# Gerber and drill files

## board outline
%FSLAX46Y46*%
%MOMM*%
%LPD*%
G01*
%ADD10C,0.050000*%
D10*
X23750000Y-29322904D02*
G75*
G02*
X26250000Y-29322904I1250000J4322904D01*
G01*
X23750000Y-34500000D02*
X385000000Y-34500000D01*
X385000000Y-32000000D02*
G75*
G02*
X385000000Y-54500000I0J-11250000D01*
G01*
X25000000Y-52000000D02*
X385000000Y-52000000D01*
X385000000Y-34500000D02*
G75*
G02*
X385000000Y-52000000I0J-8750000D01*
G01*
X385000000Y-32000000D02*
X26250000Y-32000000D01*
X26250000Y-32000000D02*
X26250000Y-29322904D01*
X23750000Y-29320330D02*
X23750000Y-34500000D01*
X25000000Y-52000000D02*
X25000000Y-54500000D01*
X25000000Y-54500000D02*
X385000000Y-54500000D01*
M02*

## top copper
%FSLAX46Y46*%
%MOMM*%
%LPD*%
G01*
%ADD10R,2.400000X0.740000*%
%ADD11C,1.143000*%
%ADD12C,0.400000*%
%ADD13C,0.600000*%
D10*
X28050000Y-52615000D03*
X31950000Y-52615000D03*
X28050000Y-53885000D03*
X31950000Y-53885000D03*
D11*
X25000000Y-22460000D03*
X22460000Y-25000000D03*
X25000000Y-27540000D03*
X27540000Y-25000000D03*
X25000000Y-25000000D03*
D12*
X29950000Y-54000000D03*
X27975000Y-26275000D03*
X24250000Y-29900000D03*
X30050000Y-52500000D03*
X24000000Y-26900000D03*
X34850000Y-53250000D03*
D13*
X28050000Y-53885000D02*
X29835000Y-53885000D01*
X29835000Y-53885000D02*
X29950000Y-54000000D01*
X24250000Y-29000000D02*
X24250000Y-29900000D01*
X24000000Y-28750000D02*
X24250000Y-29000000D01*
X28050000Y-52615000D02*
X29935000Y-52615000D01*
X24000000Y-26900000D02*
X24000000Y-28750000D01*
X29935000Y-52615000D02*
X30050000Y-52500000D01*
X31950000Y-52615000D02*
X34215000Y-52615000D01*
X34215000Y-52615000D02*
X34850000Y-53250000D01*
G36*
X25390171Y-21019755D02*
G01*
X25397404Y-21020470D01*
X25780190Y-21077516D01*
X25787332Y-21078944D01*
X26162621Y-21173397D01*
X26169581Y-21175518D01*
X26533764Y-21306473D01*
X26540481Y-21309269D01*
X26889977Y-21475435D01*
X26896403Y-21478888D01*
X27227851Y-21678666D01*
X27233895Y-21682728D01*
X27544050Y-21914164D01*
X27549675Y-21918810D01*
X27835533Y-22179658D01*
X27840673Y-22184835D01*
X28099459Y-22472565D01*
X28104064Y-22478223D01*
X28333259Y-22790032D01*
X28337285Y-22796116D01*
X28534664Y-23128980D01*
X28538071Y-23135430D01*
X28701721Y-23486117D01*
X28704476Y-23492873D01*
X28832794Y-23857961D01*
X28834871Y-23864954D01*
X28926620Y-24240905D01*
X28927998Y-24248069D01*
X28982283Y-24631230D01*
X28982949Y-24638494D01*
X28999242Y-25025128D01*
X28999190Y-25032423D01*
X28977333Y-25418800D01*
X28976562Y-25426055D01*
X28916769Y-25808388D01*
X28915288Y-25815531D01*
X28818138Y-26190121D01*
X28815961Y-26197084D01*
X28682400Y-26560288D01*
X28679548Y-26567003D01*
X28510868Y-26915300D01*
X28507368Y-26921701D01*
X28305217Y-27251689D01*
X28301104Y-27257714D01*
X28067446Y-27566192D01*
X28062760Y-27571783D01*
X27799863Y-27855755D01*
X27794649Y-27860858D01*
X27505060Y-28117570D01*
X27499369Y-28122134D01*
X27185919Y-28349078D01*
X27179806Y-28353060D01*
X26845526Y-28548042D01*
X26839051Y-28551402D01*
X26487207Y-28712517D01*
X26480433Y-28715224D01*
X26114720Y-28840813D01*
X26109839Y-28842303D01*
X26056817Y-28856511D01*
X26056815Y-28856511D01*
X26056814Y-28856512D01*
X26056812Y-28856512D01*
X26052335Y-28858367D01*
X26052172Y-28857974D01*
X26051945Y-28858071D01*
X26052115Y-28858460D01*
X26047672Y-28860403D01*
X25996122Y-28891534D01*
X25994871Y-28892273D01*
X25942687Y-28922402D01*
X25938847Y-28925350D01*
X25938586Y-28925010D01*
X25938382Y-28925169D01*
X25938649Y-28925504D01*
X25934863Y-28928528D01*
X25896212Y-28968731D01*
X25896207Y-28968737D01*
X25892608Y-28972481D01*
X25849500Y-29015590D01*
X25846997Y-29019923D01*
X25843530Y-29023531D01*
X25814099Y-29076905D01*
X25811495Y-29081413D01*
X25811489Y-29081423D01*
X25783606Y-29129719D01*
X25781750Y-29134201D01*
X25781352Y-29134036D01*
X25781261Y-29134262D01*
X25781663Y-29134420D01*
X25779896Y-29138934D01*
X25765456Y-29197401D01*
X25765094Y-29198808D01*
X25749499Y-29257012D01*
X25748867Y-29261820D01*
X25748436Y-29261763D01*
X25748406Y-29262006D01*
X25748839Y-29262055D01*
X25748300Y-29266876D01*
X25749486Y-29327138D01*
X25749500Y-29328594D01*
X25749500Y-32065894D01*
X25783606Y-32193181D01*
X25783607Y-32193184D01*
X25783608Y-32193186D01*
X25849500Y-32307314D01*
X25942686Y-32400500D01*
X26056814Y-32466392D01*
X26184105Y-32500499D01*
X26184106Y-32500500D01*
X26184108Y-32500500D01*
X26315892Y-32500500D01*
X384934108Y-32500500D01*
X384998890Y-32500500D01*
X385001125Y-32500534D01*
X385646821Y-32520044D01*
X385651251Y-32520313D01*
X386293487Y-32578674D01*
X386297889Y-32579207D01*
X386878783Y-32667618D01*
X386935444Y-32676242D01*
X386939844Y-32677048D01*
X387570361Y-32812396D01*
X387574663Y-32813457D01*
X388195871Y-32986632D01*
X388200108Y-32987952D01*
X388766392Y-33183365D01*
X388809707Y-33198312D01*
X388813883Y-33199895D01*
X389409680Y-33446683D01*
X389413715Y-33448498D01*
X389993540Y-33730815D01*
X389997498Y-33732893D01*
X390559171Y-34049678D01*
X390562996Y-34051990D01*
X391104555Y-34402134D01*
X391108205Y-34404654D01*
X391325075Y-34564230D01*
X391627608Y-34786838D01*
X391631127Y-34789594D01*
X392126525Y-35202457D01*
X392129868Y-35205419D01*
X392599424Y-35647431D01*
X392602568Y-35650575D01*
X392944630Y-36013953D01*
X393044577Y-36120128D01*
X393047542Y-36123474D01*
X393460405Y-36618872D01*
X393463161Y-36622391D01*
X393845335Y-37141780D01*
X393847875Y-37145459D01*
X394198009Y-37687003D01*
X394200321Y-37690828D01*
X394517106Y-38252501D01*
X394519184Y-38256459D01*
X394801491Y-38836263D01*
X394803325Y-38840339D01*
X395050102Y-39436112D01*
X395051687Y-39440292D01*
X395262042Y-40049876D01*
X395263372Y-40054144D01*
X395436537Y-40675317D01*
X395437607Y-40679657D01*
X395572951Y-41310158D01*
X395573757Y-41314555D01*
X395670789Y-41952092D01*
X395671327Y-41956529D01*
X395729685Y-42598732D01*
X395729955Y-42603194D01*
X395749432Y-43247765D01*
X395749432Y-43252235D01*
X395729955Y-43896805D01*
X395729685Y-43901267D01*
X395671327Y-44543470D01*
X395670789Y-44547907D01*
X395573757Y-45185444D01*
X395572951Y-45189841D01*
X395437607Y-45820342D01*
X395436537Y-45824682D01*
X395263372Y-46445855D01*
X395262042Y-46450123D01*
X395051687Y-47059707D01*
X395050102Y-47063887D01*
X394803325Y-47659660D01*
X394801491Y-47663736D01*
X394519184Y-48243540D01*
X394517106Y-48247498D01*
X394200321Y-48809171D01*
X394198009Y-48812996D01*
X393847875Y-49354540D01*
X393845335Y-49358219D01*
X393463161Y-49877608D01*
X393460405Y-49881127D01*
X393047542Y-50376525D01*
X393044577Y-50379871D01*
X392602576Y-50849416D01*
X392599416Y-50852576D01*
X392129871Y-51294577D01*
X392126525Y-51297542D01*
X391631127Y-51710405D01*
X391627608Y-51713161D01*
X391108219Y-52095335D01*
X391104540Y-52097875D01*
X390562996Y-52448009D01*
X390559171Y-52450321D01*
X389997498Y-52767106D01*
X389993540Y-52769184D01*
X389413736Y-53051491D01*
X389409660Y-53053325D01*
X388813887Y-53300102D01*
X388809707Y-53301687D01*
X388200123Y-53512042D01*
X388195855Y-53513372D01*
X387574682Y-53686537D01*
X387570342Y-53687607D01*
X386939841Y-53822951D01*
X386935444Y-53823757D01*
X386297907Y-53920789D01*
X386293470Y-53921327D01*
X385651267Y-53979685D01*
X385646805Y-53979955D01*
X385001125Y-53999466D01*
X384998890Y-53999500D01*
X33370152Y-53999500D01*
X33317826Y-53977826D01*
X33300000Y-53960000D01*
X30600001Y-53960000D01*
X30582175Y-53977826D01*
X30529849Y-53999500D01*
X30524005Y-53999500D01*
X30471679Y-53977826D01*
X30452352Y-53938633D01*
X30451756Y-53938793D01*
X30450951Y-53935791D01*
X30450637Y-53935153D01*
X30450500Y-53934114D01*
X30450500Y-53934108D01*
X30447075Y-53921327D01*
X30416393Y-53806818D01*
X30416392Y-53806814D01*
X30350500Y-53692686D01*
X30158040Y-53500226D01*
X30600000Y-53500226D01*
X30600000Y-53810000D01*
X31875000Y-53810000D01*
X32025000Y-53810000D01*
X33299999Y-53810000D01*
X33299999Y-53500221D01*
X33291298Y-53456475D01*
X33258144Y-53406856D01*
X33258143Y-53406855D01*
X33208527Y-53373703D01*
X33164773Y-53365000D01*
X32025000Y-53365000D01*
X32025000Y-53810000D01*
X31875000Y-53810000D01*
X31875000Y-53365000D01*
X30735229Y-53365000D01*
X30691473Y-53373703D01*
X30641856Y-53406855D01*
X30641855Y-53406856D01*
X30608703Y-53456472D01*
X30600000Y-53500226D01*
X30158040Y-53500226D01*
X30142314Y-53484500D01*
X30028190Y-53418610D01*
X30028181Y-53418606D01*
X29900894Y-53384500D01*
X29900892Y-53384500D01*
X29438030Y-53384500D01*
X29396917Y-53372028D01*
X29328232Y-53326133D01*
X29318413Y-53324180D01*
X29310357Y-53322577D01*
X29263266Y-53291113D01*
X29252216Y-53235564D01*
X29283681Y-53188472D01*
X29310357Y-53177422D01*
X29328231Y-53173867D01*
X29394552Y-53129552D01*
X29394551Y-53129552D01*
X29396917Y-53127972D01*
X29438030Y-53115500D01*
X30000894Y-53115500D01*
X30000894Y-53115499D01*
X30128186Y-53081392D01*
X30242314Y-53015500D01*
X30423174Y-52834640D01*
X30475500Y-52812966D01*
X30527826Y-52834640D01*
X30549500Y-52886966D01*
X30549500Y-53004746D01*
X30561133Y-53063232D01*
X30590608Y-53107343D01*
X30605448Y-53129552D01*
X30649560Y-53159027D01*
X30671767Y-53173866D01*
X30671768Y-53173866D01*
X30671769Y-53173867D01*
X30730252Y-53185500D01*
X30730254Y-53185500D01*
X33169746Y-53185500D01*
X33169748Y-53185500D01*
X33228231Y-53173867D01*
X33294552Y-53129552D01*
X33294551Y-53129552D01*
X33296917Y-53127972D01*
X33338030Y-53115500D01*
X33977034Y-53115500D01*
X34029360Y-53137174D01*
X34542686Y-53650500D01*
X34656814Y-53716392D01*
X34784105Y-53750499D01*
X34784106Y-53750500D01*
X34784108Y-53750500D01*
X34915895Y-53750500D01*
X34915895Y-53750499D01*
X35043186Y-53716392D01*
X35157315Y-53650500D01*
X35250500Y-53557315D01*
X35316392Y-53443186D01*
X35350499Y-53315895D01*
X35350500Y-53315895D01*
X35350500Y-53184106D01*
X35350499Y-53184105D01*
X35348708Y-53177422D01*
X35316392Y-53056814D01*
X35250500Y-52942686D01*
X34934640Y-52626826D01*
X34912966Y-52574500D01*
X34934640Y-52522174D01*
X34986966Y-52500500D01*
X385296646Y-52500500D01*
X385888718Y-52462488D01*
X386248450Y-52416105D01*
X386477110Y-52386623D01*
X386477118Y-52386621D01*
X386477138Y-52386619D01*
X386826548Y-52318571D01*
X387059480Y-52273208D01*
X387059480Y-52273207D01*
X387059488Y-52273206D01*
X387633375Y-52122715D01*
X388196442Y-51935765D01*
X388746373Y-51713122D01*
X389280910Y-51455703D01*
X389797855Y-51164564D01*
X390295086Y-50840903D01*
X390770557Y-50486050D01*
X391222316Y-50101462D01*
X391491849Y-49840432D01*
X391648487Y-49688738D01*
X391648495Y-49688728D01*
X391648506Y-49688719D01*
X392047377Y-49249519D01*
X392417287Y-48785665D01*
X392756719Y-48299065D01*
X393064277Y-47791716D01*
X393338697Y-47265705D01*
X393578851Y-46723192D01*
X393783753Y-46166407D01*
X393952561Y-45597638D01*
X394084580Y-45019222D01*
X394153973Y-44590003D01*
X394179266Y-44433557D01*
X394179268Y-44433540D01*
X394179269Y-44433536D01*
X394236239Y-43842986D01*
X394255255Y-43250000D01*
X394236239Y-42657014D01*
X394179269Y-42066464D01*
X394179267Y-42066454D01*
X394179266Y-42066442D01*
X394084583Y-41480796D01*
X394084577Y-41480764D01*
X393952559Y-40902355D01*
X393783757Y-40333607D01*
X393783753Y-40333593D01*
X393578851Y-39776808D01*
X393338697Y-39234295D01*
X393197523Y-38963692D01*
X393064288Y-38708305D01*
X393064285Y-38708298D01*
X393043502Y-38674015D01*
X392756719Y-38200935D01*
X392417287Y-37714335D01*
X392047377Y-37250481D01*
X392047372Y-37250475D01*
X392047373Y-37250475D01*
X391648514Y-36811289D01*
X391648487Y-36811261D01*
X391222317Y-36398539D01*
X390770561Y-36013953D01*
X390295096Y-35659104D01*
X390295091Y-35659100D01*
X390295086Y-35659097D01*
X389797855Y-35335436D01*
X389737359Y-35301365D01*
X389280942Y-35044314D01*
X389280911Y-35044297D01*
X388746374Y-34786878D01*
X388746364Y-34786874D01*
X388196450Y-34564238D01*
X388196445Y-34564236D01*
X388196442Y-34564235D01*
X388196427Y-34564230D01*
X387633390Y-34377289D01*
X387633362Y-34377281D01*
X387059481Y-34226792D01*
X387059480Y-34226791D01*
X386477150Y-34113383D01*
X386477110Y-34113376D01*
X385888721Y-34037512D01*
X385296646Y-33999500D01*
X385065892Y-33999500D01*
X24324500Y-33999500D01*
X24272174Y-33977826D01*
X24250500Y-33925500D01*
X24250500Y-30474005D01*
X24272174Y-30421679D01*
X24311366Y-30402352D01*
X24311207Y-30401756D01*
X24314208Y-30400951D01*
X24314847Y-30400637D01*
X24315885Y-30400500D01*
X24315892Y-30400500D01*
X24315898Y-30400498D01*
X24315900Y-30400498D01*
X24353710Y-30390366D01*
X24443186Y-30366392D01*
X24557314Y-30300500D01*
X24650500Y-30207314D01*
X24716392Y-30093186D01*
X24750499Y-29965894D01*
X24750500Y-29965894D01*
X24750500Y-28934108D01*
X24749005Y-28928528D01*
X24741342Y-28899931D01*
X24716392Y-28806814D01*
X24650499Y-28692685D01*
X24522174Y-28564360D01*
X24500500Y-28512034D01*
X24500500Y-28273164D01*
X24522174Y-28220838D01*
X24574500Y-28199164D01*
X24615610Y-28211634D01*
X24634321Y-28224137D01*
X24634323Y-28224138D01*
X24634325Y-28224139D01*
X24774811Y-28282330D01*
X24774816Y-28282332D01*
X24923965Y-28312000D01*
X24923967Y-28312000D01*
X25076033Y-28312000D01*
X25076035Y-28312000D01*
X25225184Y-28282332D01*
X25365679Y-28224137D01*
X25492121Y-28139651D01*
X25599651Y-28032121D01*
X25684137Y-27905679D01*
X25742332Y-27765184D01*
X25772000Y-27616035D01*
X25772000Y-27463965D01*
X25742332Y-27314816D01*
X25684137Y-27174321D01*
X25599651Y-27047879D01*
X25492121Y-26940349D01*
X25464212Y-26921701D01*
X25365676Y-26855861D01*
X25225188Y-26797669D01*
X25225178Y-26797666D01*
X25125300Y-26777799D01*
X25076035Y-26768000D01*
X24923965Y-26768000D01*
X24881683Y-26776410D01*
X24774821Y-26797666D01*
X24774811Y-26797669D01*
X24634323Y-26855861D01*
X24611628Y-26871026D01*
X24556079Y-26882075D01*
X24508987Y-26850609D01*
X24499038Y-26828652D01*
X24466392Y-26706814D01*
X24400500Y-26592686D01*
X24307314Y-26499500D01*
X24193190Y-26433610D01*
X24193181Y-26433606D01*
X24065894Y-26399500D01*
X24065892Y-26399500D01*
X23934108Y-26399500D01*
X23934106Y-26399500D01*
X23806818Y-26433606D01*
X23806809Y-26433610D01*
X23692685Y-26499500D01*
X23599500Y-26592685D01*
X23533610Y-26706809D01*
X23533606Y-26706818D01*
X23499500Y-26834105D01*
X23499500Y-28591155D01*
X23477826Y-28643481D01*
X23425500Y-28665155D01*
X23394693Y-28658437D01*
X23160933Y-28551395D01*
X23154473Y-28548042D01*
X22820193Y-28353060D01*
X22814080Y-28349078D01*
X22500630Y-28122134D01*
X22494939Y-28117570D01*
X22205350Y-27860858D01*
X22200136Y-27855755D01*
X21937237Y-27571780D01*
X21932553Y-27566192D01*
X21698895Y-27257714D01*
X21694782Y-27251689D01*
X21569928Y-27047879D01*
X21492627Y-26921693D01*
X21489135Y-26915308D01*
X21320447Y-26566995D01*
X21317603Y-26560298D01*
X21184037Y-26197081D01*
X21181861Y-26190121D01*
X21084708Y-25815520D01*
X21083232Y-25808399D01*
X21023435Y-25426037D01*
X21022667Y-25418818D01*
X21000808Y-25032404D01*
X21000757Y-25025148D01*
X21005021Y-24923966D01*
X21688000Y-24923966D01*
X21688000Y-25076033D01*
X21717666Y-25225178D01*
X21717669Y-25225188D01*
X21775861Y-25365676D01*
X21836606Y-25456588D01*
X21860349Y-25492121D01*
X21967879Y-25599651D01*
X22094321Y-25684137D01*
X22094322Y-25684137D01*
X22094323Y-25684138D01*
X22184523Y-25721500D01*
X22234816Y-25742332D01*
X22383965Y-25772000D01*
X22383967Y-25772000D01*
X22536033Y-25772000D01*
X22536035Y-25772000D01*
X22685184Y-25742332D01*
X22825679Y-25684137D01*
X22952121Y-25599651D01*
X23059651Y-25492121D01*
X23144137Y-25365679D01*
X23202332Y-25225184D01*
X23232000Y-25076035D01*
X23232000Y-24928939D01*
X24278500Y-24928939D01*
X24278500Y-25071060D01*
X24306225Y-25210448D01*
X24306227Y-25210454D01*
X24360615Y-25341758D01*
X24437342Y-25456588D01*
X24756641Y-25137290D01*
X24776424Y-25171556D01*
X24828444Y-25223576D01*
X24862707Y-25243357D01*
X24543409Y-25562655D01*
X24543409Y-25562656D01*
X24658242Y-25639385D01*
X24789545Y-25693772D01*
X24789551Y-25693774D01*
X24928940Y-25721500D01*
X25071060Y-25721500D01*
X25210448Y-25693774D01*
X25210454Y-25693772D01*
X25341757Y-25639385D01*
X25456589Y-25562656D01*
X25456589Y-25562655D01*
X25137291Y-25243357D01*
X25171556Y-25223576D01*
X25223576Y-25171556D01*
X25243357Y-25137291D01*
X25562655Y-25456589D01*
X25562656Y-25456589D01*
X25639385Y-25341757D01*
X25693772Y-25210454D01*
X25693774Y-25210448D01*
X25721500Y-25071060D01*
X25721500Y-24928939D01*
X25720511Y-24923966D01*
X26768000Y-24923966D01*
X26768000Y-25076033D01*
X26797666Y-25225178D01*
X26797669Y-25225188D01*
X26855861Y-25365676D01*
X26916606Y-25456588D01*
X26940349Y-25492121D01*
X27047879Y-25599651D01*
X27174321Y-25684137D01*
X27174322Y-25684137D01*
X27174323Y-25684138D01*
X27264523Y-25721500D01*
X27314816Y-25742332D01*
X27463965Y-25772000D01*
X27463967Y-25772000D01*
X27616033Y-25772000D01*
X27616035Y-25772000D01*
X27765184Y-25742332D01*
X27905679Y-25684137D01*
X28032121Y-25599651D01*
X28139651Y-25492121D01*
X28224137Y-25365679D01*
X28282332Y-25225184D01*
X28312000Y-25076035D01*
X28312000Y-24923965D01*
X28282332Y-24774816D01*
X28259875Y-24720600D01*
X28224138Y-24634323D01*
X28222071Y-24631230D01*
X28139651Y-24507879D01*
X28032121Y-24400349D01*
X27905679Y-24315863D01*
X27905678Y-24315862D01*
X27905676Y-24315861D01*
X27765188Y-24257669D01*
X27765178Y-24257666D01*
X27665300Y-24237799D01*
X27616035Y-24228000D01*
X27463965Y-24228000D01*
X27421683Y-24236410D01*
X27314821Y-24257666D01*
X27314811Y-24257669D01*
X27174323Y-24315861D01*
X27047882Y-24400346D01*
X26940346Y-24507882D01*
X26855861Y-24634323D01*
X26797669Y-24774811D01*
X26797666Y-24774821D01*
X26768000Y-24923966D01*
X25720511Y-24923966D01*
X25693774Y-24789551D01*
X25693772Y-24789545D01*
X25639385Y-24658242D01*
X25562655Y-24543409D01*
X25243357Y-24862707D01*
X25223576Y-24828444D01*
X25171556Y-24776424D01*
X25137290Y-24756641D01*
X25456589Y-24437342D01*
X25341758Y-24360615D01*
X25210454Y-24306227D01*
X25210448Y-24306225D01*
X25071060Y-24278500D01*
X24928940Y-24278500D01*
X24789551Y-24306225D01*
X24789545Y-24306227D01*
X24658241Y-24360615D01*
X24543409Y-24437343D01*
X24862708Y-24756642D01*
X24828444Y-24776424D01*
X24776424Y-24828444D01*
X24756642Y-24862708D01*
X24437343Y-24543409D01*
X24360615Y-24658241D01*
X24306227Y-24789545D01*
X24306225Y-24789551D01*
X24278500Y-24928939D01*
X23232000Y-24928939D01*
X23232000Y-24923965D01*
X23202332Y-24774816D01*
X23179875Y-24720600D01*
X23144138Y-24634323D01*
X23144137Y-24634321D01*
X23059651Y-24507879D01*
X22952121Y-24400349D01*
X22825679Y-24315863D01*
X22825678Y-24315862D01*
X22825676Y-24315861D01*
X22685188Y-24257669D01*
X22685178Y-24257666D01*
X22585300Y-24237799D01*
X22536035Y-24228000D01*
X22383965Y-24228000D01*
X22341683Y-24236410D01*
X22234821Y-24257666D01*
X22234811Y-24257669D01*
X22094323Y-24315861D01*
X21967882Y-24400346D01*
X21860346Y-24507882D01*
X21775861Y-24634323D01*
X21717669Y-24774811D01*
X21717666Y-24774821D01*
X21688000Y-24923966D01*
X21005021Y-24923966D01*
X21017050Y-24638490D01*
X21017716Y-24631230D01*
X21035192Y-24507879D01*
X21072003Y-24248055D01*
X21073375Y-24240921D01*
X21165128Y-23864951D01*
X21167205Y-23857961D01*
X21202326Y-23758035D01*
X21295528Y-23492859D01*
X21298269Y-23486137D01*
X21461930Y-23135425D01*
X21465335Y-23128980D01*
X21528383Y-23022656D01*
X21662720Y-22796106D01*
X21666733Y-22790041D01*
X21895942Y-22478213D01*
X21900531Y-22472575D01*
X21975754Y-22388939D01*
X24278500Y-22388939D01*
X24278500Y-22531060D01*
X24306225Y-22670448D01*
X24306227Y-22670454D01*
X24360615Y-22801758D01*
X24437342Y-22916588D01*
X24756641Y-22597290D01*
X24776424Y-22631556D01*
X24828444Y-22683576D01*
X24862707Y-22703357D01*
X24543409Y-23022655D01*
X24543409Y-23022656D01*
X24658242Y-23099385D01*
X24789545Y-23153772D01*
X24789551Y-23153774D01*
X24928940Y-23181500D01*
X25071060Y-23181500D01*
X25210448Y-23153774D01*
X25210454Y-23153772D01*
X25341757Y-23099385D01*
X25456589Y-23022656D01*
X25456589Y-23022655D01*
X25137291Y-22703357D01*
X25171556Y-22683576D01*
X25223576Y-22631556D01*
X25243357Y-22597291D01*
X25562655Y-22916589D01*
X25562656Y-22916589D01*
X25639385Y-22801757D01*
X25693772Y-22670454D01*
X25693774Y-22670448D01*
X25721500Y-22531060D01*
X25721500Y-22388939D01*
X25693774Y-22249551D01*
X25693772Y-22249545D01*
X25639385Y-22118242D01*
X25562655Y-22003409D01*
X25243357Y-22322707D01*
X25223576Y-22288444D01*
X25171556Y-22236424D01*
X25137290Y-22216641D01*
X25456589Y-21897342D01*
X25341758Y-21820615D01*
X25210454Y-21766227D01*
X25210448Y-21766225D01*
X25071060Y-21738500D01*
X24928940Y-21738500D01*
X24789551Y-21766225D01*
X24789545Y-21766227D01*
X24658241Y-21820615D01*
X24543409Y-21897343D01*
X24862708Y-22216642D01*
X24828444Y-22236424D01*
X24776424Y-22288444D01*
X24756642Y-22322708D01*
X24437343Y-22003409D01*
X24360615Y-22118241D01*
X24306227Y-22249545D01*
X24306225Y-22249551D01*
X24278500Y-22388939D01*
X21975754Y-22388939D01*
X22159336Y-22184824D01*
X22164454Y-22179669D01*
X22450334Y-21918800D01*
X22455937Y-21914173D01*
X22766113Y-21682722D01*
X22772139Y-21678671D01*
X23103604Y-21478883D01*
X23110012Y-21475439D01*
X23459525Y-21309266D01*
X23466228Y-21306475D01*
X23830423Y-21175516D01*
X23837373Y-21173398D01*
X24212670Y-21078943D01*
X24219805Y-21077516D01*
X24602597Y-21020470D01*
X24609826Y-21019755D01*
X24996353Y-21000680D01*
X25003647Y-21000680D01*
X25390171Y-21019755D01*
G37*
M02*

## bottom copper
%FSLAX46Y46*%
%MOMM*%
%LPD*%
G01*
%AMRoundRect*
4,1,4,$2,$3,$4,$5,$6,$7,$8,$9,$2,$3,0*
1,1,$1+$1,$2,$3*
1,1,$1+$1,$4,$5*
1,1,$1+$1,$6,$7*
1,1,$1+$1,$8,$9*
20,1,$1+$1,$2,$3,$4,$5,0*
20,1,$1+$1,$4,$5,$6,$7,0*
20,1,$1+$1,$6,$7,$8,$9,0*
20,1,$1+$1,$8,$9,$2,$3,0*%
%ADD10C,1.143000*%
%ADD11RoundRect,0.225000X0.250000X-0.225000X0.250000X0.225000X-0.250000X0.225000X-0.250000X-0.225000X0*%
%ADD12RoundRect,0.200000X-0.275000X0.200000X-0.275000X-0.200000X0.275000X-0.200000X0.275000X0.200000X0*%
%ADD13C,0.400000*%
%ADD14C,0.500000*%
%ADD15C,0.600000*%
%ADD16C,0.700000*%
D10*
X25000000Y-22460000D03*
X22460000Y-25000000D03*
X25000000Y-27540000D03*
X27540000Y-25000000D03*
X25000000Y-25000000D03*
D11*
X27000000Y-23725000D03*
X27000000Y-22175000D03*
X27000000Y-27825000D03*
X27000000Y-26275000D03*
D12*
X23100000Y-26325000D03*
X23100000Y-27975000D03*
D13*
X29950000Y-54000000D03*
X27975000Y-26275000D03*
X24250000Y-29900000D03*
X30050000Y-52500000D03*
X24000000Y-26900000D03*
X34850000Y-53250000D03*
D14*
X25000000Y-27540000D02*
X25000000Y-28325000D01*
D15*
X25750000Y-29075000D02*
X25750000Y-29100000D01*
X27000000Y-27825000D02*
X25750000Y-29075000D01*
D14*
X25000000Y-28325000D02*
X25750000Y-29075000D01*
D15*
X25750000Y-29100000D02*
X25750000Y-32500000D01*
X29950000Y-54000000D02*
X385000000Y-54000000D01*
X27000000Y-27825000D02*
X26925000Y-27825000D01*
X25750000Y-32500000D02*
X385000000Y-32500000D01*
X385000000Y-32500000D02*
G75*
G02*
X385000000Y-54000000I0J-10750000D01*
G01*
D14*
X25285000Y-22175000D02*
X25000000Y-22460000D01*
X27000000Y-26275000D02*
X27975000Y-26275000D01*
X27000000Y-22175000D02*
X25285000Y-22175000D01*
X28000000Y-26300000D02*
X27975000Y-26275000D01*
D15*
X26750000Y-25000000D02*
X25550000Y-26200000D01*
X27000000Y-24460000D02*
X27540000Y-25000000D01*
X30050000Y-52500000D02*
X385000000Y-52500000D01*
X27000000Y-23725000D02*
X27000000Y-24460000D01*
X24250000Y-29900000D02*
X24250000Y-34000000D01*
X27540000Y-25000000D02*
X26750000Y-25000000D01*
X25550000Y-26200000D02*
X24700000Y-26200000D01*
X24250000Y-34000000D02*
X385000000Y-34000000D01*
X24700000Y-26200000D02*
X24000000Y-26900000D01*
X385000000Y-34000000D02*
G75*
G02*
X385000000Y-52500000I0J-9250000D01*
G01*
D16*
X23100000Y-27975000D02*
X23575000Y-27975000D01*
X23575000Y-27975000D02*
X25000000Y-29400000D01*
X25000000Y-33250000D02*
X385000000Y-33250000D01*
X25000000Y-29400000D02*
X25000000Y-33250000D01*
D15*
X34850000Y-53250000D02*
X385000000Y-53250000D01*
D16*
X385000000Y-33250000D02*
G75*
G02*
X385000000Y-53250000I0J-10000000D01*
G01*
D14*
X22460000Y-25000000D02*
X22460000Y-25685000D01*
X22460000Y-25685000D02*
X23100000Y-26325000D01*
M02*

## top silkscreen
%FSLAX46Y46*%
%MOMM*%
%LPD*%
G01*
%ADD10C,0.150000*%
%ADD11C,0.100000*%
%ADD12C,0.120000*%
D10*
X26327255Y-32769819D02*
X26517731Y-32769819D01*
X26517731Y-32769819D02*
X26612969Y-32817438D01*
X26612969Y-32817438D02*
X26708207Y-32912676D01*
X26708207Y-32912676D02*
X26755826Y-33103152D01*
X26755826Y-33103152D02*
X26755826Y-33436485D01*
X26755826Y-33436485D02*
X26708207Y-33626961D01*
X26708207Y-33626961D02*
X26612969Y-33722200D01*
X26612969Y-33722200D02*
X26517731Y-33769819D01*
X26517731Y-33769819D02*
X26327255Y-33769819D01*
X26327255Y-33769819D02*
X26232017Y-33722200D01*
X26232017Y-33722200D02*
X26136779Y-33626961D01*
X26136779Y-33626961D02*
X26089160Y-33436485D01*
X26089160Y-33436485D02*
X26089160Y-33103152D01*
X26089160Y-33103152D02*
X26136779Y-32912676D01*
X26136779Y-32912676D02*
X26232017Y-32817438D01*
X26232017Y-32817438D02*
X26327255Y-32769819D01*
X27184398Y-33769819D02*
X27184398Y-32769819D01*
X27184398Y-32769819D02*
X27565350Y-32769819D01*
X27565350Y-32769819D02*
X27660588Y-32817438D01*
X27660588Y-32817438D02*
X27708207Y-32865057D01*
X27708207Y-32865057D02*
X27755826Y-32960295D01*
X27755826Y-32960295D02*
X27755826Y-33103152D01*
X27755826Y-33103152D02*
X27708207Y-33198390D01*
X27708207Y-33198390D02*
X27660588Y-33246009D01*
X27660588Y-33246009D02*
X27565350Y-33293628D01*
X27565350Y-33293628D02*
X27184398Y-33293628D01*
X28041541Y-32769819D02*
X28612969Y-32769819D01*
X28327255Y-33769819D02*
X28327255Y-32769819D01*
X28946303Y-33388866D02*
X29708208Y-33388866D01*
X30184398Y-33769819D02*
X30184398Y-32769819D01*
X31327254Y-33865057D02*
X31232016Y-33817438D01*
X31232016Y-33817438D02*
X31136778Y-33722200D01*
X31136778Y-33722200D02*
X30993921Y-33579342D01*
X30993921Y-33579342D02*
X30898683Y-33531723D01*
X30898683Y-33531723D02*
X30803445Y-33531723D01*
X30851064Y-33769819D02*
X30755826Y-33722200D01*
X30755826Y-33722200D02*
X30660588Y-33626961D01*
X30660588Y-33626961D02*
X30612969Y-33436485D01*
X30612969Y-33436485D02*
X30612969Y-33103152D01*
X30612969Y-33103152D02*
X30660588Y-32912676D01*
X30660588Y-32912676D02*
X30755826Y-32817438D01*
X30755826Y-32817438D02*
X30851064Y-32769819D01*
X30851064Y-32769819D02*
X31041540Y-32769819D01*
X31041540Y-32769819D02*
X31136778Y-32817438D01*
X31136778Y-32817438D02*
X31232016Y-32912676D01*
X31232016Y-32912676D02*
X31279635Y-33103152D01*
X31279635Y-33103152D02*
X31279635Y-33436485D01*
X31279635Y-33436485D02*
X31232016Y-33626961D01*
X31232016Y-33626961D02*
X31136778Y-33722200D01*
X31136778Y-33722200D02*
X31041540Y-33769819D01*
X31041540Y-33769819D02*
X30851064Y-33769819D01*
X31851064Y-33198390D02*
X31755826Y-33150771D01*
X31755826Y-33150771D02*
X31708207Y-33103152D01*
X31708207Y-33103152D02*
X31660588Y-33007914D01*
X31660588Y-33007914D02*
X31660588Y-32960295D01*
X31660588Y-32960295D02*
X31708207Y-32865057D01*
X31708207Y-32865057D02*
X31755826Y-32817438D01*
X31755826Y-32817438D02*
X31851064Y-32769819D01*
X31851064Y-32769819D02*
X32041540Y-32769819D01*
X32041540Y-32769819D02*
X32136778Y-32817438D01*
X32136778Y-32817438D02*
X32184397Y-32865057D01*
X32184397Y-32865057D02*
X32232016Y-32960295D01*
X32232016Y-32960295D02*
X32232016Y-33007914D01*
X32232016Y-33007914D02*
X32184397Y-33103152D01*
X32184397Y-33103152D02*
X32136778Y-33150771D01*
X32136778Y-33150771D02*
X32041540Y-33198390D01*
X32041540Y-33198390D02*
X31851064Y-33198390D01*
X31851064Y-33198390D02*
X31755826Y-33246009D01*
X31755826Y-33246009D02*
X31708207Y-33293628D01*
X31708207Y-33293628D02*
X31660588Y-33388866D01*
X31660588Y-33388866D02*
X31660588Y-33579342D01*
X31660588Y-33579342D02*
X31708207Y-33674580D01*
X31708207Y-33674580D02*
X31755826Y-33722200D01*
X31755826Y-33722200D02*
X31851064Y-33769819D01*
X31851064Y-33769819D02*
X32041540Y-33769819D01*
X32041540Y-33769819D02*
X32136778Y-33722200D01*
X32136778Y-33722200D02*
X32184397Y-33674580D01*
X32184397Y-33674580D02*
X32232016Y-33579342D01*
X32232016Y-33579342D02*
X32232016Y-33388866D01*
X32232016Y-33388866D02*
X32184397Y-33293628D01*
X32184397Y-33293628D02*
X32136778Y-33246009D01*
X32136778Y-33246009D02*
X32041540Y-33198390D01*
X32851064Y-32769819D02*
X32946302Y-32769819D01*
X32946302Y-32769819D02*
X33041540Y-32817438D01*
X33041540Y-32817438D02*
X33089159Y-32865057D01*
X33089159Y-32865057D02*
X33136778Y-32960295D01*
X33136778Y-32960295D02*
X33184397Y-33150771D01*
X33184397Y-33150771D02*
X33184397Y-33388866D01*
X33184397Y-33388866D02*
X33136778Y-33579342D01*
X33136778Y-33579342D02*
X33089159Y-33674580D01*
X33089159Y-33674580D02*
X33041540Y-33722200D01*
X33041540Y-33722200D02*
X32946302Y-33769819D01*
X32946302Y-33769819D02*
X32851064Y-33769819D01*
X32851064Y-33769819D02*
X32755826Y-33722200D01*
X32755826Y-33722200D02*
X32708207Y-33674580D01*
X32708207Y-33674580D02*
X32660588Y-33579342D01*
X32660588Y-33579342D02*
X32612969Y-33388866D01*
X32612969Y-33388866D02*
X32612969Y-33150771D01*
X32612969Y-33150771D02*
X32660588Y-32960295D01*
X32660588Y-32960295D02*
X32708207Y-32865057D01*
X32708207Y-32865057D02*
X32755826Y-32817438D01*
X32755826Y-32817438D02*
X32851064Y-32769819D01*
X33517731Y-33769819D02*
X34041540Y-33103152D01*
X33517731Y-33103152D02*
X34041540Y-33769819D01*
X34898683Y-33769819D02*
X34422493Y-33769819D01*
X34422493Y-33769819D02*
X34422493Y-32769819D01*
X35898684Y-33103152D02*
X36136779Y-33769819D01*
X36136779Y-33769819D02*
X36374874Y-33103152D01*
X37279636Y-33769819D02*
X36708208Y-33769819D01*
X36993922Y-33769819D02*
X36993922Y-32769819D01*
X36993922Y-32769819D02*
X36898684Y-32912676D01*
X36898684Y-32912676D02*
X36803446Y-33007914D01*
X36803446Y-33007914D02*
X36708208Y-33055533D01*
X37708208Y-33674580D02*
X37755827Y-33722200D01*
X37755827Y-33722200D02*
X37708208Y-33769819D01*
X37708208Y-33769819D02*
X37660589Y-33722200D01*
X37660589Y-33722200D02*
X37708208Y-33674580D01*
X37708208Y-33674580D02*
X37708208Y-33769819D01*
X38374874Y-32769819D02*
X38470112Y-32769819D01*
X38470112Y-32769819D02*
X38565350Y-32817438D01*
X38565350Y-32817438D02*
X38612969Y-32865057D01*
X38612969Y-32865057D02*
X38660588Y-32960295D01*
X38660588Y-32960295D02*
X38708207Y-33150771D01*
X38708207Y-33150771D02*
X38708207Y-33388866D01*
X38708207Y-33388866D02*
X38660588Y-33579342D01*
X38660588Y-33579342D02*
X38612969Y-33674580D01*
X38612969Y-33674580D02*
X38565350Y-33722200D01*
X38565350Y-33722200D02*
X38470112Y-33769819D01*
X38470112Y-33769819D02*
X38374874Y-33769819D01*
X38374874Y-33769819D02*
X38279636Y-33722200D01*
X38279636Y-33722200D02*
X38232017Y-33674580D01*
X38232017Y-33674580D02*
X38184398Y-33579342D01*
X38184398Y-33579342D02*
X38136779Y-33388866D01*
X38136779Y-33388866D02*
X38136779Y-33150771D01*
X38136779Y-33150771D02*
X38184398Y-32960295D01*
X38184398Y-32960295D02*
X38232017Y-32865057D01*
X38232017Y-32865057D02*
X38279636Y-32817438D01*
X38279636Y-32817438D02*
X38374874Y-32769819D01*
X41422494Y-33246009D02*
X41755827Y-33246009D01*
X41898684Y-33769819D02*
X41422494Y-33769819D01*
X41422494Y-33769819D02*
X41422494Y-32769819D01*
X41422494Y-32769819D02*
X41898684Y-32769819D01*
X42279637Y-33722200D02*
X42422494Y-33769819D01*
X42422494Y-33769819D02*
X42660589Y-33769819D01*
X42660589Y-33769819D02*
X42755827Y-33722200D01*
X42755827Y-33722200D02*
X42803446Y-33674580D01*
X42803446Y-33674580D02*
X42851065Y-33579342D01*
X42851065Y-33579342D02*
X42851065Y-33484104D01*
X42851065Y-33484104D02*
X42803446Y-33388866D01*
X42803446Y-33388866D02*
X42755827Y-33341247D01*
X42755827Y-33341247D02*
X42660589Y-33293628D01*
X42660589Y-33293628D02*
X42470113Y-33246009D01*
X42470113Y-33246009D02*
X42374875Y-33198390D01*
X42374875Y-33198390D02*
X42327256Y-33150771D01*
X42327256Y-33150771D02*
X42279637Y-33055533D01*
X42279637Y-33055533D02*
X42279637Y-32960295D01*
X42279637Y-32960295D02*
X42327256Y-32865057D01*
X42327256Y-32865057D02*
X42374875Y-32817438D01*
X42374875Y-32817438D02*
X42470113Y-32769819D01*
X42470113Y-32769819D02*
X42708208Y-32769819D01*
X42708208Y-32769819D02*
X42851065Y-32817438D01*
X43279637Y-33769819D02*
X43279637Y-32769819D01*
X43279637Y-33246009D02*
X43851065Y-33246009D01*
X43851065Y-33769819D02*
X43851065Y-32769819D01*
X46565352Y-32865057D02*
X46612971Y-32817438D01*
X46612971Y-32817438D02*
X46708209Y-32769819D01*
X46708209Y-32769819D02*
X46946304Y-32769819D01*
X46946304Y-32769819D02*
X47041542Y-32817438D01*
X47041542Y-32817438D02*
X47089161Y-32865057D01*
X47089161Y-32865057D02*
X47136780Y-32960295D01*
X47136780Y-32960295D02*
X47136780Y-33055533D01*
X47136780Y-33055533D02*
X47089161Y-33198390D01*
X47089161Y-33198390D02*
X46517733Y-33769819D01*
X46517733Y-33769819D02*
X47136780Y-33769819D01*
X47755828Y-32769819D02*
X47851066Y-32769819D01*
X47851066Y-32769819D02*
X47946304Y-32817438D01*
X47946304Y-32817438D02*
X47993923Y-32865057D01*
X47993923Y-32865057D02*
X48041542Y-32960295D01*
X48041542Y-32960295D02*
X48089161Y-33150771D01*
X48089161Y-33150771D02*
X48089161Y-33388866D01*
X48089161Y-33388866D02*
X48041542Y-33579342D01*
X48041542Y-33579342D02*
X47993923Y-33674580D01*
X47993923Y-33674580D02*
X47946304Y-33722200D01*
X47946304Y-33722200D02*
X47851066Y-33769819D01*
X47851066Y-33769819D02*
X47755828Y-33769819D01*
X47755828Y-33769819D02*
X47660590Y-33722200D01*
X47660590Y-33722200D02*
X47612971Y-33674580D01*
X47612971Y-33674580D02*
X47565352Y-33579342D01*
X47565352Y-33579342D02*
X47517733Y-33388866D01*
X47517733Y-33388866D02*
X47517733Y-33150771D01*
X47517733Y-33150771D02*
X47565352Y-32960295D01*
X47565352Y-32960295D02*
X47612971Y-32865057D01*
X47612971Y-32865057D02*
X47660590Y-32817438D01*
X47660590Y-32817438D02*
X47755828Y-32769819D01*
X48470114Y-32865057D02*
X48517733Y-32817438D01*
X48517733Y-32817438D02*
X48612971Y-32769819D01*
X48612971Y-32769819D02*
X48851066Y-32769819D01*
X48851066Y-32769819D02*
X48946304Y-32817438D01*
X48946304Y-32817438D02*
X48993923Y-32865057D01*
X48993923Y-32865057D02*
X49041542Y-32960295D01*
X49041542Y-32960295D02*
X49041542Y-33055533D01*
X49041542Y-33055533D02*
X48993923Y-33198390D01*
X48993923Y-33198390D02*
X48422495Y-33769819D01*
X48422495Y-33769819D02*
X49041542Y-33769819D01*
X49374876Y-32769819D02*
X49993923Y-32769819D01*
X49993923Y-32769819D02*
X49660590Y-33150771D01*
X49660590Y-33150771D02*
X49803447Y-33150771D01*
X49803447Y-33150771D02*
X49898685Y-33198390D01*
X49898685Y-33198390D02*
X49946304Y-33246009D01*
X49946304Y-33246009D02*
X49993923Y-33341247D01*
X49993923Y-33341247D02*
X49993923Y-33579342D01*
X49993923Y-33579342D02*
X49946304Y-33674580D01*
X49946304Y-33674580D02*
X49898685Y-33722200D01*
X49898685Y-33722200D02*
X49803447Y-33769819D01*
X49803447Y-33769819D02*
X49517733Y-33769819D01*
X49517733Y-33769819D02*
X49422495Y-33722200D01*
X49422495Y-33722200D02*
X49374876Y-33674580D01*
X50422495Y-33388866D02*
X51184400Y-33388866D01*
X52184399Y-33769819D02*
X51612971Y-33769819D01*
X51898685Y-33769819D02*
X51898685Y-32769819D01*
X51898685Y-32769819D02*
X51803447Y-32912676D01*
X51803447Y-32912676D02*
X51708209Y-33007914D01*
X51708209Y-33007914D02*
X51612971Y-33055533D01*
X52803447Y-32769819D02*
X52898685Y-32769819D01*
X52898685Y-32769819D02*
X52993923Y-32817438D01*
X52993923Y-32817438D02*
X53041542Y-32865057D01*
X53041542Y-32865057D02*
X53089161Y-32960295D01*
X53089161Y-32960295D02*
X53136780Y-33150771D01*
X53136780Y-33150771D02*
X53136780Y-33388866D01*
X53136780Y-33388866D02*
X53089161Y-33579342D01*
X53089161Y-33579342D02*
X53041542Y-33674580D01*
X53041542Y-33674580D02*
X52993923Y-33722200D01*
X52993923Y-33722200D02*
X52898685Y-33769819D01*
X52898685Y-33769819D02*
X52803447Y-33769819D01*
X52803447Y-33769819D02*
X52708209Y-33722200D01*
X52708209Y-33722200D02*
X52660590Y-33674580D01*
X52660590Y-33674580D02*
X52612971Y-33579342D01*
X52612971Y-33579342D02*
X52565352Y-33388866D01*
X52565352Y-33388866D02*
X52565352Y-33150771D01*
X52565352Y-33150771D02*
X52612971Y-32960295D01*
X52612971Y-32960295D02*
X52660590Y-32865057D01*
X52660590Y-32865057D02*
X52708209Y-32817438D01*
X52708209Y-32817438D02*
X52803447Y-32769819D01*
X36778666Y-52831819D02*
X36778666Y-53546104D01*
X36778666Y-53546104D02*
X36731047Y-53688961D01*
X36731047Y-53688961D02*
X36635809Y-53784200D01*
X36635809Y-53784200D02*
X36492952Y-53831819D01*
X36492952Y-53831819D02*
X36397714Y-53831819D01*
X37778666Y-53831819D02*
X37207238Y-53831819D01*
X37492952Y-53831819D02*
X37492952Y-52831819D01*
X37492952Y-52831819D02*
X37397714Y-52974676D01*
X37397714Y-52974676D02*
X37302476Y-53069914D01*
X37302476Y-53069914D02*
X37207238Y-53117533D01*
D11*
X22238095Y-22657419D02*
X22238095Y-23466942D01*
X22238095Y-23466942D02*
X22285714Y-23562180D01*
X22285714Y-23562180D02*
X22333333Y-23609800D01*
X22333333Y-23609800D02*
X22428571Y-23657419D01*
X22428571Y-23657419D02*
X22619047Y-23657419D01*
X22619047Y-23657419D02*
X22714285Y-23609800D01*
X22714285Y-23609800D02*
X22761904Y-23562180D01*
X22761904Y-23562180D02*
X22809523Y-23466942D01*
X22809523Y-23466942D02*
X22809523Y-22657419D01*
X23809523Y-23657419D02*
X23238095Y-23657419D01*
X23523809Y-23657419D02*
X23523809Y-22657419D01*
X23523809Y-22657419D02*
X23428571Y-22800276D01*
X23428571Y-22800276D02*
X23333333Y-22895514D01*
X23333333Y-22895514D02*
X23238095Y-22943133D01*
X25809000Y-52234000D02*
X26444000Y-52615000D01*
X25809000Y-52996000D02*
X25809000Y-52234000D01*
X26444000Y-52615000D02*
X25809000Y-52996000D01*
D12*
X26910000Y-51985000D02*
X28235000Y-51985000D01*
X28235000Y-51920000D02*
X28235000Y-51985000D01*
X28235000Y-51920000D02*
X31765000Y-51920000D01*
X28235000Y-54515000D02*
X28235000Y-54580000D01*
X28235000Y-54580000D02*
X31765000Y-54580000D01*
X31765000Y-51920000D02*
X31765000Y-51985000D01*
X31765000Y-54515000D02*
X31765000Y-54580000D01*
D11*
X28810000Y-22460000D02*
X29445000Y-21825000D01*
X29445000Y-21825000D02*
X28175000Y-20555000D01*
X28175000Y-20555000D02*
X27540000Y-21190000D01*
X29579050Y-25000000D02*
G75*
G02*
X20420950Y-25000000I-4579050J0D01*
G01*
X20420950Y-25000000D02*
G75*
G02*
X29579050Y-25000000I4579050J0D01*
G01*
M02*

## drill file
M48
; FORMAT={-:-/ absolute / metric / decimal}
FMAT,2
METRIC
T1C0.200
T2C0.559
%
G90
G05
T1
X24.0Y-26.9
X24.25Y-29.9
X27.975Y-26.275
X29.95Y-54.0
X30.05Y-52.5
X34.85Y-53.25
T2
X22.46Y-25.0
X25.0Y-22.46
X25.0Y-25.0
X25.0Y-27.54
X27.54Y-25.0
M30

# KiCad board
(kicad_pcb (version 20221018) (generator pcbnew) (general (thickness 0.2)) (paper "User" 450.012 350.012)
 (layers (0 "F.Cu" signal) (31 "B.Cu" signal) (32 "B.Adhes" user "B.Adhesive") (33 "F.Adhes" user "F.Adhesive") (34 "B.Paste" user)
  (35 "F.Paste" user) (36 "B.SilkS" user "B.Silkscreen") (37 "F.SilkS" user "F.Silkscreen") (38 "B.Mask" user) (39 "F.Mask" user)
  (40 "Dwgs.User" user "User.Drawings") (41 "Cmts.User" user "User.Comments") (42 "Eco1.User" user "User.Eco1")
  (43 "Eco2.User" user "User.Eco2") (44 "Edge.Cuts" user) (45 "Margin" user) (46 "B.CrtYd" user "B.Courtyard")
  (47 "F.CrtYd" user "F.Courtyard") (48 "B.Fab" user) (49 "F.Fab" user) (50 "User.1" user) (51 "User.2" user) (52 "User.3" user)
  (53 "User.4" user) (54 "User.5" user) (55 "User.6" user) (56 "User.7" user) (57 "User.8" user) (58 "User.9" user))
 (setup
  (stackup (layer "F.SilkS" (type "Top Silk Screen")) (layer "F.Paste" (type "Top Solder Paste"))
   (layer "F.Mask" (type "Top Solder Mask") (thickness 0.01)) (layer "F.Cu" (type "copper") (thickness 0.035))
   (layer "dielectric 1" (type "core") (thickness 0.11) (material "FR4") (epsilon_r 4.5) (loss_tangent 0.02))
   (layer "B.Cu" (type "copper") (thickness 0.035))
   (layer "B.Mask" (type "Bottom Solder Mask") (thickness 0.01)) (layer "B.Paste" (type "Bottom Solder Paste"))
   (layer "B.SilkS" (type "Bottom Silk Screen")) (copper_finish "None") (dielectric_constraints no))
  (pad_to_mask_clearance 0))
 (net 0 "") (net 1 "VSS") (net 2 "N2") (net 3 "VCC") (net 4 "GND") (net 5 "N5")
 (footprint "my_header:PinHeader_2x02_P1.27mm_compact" (layer "F.Cu") (at 30 53.25)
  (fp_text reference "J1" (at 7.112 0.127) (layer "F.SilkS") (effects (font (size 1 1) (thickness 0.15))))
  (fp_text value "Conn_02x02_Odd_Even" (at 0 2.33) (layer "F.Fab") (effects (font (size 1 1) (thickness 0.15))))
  (fp_line (start -4.191 -1.016) (end -3.556 -0.635) (stroke (width 0.1) (type default)) (layer "F.SilkS"))
  (fp_line (start -4.191 -0.254) (end -4.191 -1.016) (stroke (width 0.1) (type default)) (layer "F.SilkS"))
  (fp_line (start -3.556 -0.635) (end -4.191 -0.254) (stroke (width 0.1) (type default)) (layer "F.SilkS"))
  (fp_line (start -3.09 -1.265) (end -1.765 -1.265) (stroke (width 0.12) (type solid)) (layer "F.SilkS"))
  (fp_line (start -1.765 -1.33) (end -1.765 -1.265) (stroke (width 0.12) (type solid)) (layer "F.SilkS"))
  (fp_line (start -1.765 -1.33) (end 1.765 -1.33) (stroke (width 0.12) (type solid)) (layer "F.SilkS"))
  (fp_line (start -1.765 1.265) (end -1.765 1.33) (stroke (width 0.12) (type solid)) (layer "F.SilkS"))
  (fp_line (start -1.765 1.33) (end 1.765 1.33) (stroke (width 0.12) (type solid)) (layer "F.SilkS"))
  (fp_line (start 1.765 -1.33) (end 1.765 -1.265) (stroke (width 0.12) (type solid)) (layer "F.SilkS"))
  (fp_line (start 1.765 1.265) (end 1.765 1.33) (stroke (width 0.12) (type solid)) (layer "F.SilkS"))
  (pad "1" smd rect (at -1.95 -0.635) (size 2.4 0.74) (layers "F.Cu" "F.Paste" "F.Mask") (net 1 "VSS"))
  (pad "2" smd rect (at 1.95 -0.635) (size 2.4 0.74) (layers "F.Cu" "F.Paste" "F.Mask") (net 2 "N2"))
  (pad "3" smd rect (at -1.95 0.635) (size 2.4 0.74) (layers "F.Cu" "F.Paste" "F.Mask") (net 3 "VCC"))
  (pad "4" smd rect (at 1.95 0.635) (size 2.4 0.74) (layers "F.Cu" "F.Paste" "F.Mask") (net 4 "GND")))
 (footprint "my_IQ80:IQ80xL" (layer "F.Cu") (at 25 25 90)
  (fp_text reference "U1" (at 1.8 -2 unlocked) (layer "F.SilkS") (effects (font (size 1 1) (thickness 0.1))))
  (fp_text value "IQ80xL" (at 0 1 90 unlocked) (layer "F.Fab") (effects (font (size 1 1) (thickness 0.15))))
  (fp_line (start 2.54 3.81) (end 3.175 4.445) (stroke (width 0.1) (type default)) (layer "F.SilkS"))
  (fp_line (start 3.175 4.445) (end 4.445 3.175) (stroke (width 0.1) (type default)) (layer "F.SilkS"))
  (fp_line (start 4.445 3.175) (end 3.81 2.54) (stroke (width 0.1) (type default)) (layer "F.SilkS"))
  (fp_circle (center 0 0) (end 3.81 2.54) (stroke (width 0.1) (type default)) (fill none) (layer "F.SilkS"))
  (pad "1" thru_hole circle (at 2.54 0 90) (size 1.143 1.143) (drill 0.5588) (layers "*.Cu" "*.Mask") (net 4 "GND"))
  (pad "2" thru_hole circle (at 0 -2.54 90) (size 1.143 1.143) (drill 0.5588) (layers "*.Cu" "*.Mask") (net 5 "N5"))
  (pad "3" thru_hole circle (at -2.54 0 90) (size 1.143 1.143) (drill 0.5588) (layers "*.Cu" "*.Mask") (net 3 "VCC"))
  (pad "4" thru_hole circle (at 0 2.54 90) (size 1.143 1.143) (drill 0.5588) (layers "*.Cu" "*.Mask") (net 1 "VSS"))
  (pad "5" thru_hole circle (at 0 0 90) (size 1.143 1.143) (drill 0.5588) (layers "*.Cu" "*.Mask") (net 4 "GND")))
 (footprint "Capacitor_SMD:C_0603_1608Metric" (layer "B.Cu") (at 27 22.95 90)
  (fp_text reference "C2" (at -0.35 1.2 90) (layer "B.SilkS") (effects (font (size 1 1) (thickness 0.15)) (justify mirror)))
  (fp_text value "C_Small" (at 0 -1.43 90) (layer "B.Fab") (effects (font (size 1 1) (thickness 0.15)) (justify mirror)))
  (pad "1" smd roundrect (at -0.775 0 90) (size 0.9 0.95) (layers "B.Cu" "B.Paste" "B.Mask") (roundrect_rratio 0.25) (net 1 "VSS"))
  (pad "2" smd roundrect (at 0.775 0 90) (size 0.9 0.95) (layers "B.Cu" "B.Paste" "B.Mask") (roundrect_rratio 0.25) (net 4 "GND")))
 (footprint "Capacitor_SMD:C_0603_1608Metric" (layer "B.Cu") (at 27 27.05 90)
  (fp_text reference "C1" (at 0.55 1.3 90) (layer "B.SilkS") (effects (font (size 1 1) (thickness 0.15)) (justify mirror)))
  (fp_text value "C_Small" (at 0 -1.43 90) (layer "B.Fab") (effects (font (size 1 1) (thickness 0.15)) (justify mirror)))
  (pad "1" smd roundrect (at -0.775 0 90) (size 0.9 0.95) (layers "B.Cu" "B.Paste" "B.Mask") (roundrect_rratio 0.25) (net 3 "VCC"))
  (pad "2" smd roundrect (at 0.775 0 90) (size 0.9 0.95) (layers "B.Cu" "B.Paste" "B.Mask") (roundrect_rratio 0.25) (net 4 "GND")))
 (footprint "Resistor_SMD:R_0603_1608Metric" (layer "B.Cu") (at 23.1 27.15 -90)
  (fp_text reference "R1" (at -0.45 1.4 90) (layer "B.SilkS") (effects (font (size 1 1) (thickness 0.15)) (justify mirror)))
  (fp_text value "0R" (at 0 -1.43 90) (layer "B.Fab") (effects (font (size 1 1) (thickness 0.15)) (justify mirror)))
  (pad "1" smd roundrect (at -0.825 0 270) (size 0.8 0.95) (layers "B.Cu" "B.Paste" "B.Mask") (roundrect_rratio 0.25) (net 5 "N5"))
  (pad "2" smd roundrect (at 0.825 0 270) (size 0.8 0.95) (layers "B.Cu" "B.Paste" "B.Mask") (roundrect_rratio 0.25) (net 2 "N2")))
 (gr_arc (start 23.75 29.322904) (mid 25 20.5) (end 26.25 29.322904) (stroke (width 0.05) (type solid)) (layer "Edge.Cuts"))
 (gr_line (start 23.75 34.5) (end 385 34.5) (stroke (width 0.05) (type solid)) (layer "Edge.Cuts"))
 (gr_arc (start 385 32) (mid 396.25 43.25) (end 385 54.5) (stroke (width 0.05) (type solid)) (layer "Edge.Cuts"))
 (gr_line (start 25 52) (end 385 52) (stroke (width 0.05) (type solid)) (layer "Edge.Cuts"))
 (gr_arc (start 385 34.5) (mid 393.75 43.25) (end 385 52) (stroke (width 0.05) (type solid)) (layer "Edge.Cuts"))
 (gr_line (start 385 32) (end 26.25 32) (stroke (width 0.05) (type solid)) (layer "Edge.Cuts"))
 (gr_line (start 26.25 32) (end 26.25 29.322904) (stroke (width 0.05) (type solid)) (layer "Edge.Cuts"))
 (gr_line (start 23.75 29.32033) (end 23.75 34.5) (stroke (width 0.05) (type solid)) (layer "Edge.Cuts"))
 (gr_line (start 25 52) (end 25 54.5) (stroke (width 0.05) (type solid)) (layer "Edge.Cuts"))
 (gr_line (start 25 54.5) (end 385 54.5) (stroke (width 0.05) (type solid)) (layer "Edge.Cuts"))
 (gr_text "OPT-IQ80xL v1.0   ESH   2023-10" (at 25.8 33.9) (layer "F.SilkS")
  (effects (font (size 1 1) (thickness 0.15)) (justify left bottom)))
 (segment (start 28.05 53.885) (end 29.835 53.885) (width 0.6) (layer "F.Cu") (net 3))
 (segment (start 29.835 53.885) (end 29.95 54) (width 0.6) (layer "F.Cu") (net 3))
 (via (at 29.95 54) (size 0.4) (drill 0.2) (layers "F.Cu" "B.Cu") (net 3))
 (segment (start 25 27.54) (end 25 28.325) (width 0.5) (layer "B.Cu") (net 3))
 (segment (start 25.75 29.075) (end 25.75 29.1) (width 0.6) (layer "B.Cu") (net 3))
 (segment (start 27 27.825) (end 25.75 29.075) (width 0.6) (layer "B.Cu") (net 3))
 (segment (start 25 28.325) (end 25.75 29.075) (width 0.5) (layer "B.Cu") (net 3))
 (segment (start 25.75 29.1) (end 25.75 32.5) (width 0.6) (layer "B.Cu") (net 3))
 (segment (start 29.95 54) (end 385 54) (width 0.6) (layer "B.Cu") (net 3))
 (segment (start 27 27.825) (end 26.925 27.825) (width 0.6) (layer "B.Cu") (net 3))
 (segment (start 25.75 32.5) (end 385 32.5) (width 0.6) (layer "B.Cu") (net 3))
 (arc (start 385 32.5) (mid 395.75 43.25) (end 385 54) (width 0.6) (layer "B.Cu") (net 3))
 (via (at 27.975 26.275) (size 0.4) (drill 0.2) (layers "F.Cu" "B.Cu") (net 4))
 (segment (start 25.285 22.175) (end 25 22.46) (width 0.5) (layer "B.Cu") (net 4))
 (segment (start 27 26.275) (end 27.975 26.275) (width 0.5) (layer "B.Cu") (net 4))
 (segment (start 27 22.175) (end 25.285 22.175) (width 0.5) (layer "B.Cu") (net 4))
 (segment (start 28 26.3) (end 27.975 26.275) (width 0.5) (layer "B.Cu") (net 4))
 (segment (start 24.25 29) (end 24.25 29.9) (width 0.6) (layer "F.Cu") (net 1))
 (segment (start 24 28.75) (end 24.25 29) (width 0.6) (layer "F.Cu") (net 1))
 (segment (start 28.05 52.615) (end 29.935 52.615) (width 0.6) (layer "F.Cu") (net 1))
 (segment (start 24 26.9) (end 24 28.75) (width 0.6) (layer "F.Cu") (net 1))
 (segment (start 29.935 52.615) (end 30.05 52.5) (width 0.6) (layer "F.Cu") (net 1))
 (via (at 24.25 29.9) (size 0.4) (drill 0.2) (layers "F.Cu" "B.Cu") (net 1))
 (via (at 30.05 52.5) (size 0.4) (drill 0.2) (layers "F.Cu" "B.Cu") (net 1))
 (via (at 24 26.9) (size 0.4) (drill 0.2) (layers "F.Cu" "B.Cu") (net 1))
 (segment (start 26.75 25) (end 25.55 26.2) (width 0.6) (layer "B.Cu") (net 1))
 (segment (start 27 24.46) (end 27.54 25) (width 0.6) (layer "B.Cu") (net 1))
 (segment (start 30.05 52.5) (end 385 52.5) (width 0.6) (layer "B.Cu") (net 1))
 (segment (start 27 23.725) (end 27 24.46) (width 0.6) (layer "B.Cu") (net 1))
 (segment (start 24.25 29.9) (end 24.25 34) (width 0.6) (layer "B.Cu") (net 1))
 (segment (start 27.54 25) (end 26.75 25) (width 0.6) (layer "B.Cu") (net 1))
 (segment (start 25.55 26.2) (end 24.7 26.2) (width 0.6) (layer "B.Cu") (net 1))
 (segment (start 24.25 34) (end 385 34) (width 0.6) (layer "B.Cu") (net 1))
 (segment (start 24.7 26.2) (end 24 26.9) (width 0.6) (layer "B.Cu") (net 1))
 (arc (start 385 34) (mid 394.25 43.25) (end 385 52.5) (width 0.6) (layer "B.Cu") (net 1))
 (segment (start 31.95 52.615) (end 34.215 52.615) (width 0.6) (layer "F.Cu") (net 2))
 (segment (start 34.215 52.615) (end 34.85 53.25) (width 0.6) (layer "F.Cu") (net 2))
 (via (at 34.85 53.25) (size 0.4) (drill 0.2) (layers "F.Cu" "B.Cu") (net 2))
 (segment (start 23.1 27.975) (end 23.575 27.975) (width 0.7) (layer "B.Cu") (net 2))
 (segment (start 23.575 27.975) (end 25 29.4) (width 0.7) (layer "B.Cu") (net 2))
 (segment (start 25 33.25) (end 385 33.25) (width 0.7) (layer "B.Cu") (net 2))
 (segment (start 25 29.4) (end 25 33.25) (width 0.7) (layer "B.Cu") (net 2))
 (segment (start 34.85 53.25) (end 385 53.25) (width 0.6) (layer "B.Cu") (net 2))
 (arc (start 385 33.25) (mid 395 43.25) (end 385 53.25) (width 0.7) (layer "B.Cu") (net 2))
 (segment (start 22.46 25) (end 22.46 25.685) (width 0.5) (layer "B.Cu") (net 5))
 (segment (start 22.46 25.685) (end 23.1 26.325) (width 0.5) (layer "B.Cu") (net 5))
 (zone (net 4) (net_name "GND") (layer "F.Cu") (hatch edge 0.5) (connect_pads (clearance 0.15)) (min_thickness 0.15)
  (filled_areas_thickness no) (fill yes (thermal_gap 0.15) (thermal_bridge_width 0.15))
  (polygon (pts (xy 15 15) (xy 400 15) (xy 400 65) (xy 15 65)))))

